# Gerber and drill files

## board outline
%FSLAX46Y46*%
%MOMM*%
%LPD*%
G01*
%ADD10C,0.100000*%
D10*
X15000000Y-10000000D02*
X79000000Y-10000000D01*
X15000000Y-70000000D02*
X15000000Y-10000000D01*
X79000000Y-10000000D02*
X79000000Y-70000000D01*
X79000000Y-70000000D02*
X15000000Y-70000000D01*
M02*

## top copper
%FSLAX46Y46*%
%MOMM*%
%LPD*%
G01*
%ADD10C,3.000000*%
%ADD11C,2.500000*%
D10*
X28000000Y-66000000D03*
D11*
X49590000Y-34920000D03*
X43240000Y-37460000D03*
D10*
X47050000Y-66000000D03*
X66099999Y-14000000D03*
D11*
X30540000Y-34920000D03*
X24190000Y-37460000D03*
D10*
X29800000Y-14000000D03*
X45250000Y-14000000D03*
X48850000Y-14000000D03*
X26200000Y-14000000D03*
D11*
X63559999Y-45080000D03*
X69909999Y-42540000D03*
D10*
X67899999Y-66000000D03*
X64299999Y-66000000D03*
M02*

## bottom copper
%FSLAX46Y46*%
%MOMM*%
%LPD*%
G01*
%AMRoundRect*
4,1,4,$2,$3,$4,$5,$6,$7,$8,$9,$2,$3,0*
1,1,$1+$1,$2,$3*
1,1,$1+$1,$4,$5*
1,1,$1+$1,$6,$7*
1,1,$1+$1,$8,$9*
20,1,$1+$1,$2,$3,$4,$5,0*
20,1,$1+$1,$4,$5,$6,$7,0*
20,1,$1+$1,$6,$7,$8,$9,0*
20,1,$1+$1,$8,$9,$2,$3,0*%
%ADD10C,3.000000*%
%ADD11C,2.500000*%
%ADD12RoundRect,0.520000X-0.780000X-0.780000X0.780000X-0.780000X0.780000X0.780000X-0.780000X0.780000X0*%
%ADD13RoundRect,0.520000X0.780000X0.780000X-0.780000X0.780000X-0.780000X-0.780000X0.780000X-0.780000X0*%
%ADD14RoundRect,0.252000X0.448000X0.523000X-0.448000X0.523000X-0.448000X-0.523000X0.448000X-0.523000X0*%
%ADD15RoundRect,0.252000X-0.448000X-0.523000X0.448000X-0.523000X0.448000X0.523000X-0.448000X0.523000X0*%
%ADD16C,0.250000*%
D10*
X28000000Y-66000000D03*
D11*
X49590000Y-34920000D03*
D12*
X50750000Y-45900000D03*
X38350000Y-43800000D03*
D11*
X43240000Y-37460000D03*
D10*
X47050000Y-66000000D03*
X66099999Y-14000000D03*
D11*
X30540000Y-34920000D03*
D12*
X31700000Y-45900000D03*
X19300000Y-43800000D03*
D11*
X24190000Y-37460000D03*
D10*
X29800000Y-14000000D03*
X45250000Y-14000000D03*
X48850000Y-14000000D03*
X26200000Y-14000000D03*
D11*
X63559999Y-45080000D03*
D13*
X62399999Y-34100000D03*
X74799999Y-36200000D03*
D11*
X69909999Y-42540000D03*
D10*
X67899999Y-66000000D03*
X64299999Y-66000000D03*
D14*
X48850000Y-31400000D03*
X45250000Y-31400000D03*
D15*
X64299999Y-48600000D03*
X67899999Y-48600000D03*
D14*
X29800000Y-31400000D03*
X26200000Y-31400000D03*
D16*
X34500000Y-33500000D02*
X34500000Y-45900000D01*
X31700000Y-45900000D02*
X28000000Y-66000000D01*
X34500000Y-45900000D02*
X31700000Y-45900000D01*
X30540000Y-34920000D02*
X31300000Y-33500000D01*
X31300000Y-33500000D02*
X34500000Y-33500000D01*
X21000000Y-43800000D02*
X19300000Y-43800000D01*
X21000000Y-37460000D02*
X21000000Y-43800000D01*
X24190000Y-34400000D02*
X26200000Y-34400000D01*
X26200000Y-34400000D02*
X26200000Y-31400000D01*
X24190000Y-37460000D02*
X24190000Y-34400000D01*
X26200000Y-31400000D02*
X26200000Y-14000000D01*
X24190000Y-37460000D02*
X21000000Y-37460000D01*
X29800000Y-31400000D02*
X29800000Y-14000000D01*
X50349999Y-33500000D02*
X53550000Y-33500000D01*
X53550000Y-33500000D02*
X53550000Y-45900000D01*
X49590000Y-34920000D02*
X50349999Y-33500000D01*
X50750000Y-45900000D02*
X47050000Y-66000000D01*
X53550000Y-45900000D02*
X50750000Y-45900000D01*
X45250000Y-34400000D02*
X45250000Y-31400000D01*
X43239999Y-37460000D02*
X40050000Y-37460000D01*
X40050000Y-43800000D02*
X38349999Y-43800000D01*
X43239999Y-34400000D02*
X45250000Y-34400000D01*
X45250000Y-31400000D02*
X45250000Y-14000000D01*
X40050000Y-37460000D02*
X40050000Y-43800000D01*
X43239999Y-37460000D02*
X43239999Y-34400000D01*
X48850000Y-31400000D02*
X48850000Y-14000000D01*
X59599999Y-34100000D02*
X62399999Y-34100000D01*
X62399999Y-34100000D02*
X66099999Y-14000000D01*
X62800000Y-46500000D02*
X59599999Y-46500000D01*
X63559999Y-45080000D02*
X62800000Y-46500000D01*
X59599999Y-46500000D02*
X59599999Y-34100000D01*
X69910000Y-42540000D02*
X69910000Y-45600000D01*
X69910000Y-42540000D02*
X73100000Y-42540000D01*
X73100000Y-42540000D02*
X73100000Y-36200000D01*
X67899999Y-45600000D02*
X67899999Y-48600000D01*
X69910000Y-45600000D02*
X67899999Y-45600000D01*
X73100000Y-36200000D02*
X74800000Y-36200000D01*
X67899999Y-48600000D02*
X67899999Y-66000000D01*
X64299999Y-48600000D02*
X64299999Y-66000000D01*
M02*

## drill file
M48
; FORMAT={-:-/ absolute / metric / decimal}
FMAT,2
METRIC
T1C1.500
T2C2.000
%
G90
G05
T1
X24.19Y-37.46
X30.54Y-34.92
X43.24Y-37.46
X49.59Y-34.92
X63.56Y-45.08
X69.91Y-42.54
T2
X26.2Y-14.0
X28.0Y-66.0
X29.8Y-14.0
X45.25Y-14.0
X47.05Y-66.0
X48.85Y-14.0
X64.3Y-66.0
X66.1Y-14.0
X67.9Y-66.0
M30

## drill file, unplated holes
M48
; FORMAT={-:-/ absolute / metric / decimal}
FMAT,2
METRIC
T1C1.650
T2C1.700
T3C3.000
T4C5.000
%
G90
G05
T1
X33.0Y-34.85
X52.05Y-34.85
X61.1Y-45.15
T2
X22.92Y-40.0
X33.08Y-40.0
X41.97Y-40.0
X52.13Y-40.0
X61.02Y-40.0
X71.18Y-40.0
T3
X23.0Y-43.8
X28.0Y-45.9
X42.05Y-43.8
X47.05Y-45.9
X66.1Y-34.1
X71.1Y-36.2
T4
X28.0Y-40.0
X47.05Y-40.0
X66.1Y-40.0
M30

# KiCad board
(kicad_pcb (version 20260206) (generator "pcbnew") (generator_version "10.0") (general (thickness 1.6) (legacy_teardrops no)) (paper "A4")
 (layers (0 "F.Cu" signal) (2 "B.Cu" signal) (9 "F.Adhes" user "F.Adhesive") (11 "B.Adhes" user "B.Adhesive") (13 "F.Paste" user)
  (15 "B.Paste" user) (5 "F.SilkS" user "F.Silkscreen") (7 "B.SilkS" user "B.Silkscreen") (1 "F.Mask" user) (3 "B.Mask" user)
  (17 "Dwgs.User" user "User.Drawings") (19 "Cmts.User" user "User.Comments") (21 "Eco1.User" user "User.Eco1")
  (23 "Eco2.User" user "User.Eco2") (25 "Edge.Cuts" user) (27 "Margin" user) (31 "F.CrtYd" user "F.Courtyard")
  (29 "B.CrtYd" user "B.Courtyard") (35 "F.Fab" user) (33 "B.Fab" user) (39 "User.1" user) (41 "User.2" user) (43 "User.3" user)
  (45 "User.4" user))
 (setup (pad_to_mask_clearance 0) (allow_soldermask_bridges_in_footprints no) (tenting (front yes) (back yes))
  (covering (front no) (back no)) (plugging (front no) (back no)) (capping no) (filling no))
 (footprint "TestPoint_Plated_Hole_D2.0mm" (layer "F.Cu") (at 28 66)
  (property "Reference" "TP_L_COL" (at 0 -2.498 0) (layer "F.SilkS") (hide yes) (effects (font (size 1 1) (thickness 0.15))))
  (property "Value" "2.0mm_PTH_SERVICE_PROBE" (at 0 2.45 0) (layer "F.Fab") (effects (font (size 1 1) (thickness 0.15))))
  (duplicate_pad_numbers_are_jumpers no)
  (pad "1" thru_hole circle (at 0 0) (size 3 3) (drill 2) (layers "*.Cu" "*.Mask") (remove_unused_layers no) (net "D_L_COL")))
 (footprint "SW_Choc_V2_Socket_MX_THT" (layer "F.Cu") (at 47.05 40)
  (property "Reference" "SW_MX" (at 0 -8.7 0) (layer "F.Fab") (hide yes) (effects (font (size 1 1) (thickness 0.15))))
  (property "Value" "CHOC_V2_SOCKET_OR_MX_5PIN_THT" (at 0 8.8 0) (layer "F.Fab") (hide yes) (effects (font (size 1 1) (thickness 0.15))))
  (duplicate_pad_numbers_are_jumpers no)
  (pad "" np_thru_hole circle (at -5.08 0) (size 1.7 1.7) (drill 1.7) (layers "*.Cu" "*.Mask"))
  (pad "" np_thru_hole circle (at -5 3.8) (size 3 3) (drill 3) (layers "*.Cu" "*.Mask"))
  (pad "" np_thru_hole circle (at 0 0) (size 5 5) (drill 5) (layers "*.Cu" "*.Mask"))
  (pad "" np_thru_hole circle (at 0 5.9) (size 3 3) (drill 3) (layers "*.Cu" "*.Mask"))
  (pad "" np_thru_hole circle (at 5 -5.15) (size 1.65 1.65) (drill 1.65) (layers "*.Cu" "*.Mask"))
  (pad "" np_thru_hole circle (at 5.08 0) (size 1.7 1.7) (drill 1.7) (layers "*.Cu" "*.Mask"))
  (pad "1" thru_hole circle (at 2.54 -5.08) (size 2.5 2.5) (drill 1.5) (layers "*.Cu" "*.Mask") (remove_unused_layers no) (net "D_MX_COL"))
  (pad "1" smd roundrect (at 3.7 5.9) (size 2.6 2.6) (layers "B.Cu" "B.Mask" "B.Paste") (roundrect_rratio 0.2) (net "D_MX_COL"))
  (pad "2" smd roundrect (at -8.7 3.8) (size 2.6 2.6) (layers "B.Cu" "B.Mask" "B.Paste") (roundrect_rratio 0.2) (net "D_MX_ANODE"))
  (pad "2" thru_hole circle (at -3.81 -2.54) (size 2.5 2.5) (drill 1.5) (layers "*.Cu" "*.Mask") (remove_unused_layers no)
   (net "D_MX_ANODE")))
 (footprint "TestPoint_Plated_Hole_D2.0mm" (layer "F.Cu") (at 47.05 66)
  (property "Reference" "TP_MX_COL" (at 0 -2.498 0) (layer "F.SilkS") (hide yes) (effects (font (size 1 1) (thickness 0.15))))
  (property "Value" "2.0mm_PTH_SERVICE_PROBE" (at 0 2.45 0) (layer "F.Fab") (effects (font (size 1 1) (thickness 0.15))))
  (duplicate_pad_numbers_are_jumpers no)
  (pad "1" thru_hole circle (at 0 0) (size 3 3) (drill 2) (layers "*.Cu" "*.Mask") (remove_unused_layers no) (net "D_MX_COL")))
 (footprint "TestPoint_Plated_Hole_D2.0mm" (layer "F.Cu") (at 66.099999 14)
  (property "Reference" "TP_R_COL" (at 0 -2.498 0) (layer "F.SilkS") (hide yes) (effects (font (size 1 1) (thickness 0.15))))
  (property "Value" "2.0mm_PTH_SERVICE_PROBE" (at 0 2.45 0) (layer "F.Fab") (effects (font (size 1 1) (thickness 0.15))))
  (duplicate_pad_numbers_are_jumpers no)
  (pad "1" thru_hole circle (at 0 0) (size 3 3) (drill 2) (layers "*.Cu" "*.Mask") (remove_unused_layers no) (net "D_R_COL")))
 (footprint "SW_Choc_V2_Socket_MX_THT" (layer "F.Cu") (at 28 40)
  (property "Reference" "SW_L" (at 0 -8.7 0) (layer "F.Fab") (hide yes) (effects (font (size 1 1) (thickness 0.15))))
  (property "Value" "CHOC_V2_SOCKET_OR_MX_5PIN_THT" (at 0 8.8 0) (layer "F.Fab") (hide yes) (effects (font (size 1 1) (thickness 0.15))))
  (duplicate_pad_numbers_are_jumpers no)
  (pad "" np_thru_hole circle (at -5.08 0) (size 1.7 1.7) (drill 1.7) (layers "*.Cu" "*.Mask"))
  (pad "" np_thru_hole circle (at -5 3.8) (size 3 3) (drill 3) (layers "*.Cu" "*.Mask"))
  (pad "" np_thru_hole circle (at 0 0) (size 5 5) (drill 5) (layers "*.Cu" "*.Mask"))
  (pad "" np_thru_hole circle (at 0 5.9) (size 3 3) (drill 3) (layers "*.Cu" "*.Mask"))
  (pad "" np_thru_hole circle (at 5 -5.15) (size 1.65 1.65) (drill 1.65) (layers "*.Cu" "*.Mask"))
  (pad "" np_thru_hole circle (at 5.08 0) (size 1.7 1.7) (drill 1.7) (layers "*.Cu" "*.Mask"))
  (pad "1" thru_hole circle (at 2.54 -5.08) (size 2.5 2.5) (drill 1.5) (layers "*.Cu" "*.Mask") (remove_unused_layers no) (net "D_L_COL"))
  (pad "1" smd roundrect (at 3.7 5.9) (size 2.6 2.6) (layers "B.Cu" "B.Mask" "B.Paste") (roundrect_rratio 0.2) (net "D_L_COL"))
  (pad "2" smd roundrect (at -8.7 3.8) (size 2.6 2.6) (layers "B.Cu" "B.Mask" "B.Paste") (roundrect_rratio 0.2) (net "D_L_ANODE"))
  (pad "2" thru_hole circle (at -3.81 -2.54) (size 2.5 2.5) (drill 1.5) (layers "*.Cu" "*.Mask") (remove_unused_layers no) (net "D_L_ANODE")))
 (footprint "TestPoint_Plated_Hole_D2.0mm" (layer "F.Cu") (at 29.8 14)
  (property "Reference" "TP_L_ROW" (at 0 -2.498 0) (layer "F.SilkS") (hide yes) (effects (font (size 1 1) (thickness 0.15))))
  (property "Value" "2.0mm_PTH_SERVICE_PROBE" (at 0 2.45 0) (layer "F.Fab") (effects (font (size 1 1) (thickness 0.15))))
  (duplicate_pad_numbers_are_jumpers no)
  (pad "1" thru_hole circle (at 0 0) (size 3 3) (drill 2) (layers "*.Cu" "*.Mask") (remove_unused_layers no) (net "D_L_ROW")))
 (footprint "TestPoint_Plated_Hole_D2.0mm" (layer "F.Cu") (at 45.25 14)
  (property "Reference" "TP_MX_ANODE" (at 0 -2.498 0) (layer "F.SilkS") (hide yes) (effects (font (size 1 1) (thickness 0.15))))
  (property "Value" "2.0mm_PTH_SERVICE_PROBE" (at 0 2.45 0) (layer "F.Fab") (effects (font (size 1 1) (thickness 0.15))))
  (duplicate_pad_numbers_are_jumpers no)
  (pad "1" thru_hole circle (at 0 0) (size 3 3) (drill 2) (layers "*.Cu" "*.Mask") (remove_unused_layers no) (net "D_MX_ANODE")))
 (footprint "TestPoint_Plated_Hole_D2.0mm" (layer "F.Cu") (at 48.85 14)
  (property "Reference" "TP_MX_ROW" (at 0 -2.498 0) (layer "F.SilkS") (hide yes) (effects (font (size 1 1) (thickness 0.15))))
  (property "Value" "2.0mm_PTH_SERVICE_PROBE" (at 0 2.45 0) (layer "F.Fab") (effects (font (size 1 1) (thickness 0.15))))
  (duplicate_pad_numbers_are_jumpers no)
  (pad "1" thru_hole circle (at 0 0) (size 3 3) (drill 2) (layers "*.Cu" "*.Mask") (remove_unused_layers no) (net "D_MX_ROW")))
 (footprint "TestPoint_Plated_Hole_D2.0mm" (layer "F.Cu") (at 26.2 14)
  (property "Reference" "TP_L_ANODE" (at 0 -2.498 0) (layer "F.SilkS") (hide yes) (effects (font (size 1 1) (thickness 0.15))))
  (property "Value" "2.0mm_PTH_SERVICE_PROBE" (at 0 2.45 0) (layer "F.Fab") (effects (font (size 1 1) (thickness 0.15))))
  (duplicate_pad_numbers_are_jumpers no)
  (pad "1" thru_hole circle (at 0 0) (size 3 3) (drill 2) (layers "*.Cu" "*.Mask") (remove_unused_layers no) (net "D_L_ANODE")))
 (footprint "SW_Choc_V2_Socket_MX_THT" (layer "F.Cu") (at 66.099999 40 180)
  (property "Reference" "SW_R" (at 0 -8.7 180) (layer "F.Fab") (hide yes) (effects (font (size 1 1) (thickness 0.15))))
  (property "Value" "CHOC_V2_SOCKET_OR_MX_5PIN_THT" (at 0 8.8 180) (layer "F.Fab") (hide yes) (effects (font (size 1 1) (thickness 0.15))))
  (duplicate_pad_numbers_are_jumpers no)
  (pad "" np_thru_hole circle (at -5.08 0 180) (size 1.7 1.7) (drill 1.7) (layers "*.Cu" "*.Mask"))
  (pad "" np_thru_hole circle (at -5 3.8 180) (size 3 3) (drill 3) (layers "*.Cu" "*.Mask"))
  (pad "" np_thru_hole circle (at 0 0 180) (size 5 5) (drill 5) (layers "*.Cu" "*.Mask"))
  (pad "" np_thru_hole circle (at 0 5.9 180) (size 3 3) (drill 3) (layers "*.Cu" "*.Mask"))
  (pad "" np_thru_hole circle (at 5 -5.15 180) (size 1.65 1.65) (drill 1.65) (layers "*.Cu" "*.Mask"))
  (pad "" np_thru_hole circle (at 5.08 0 180) (size 1.7 1.7) (drill 1.7) (layers "*.Cu" "*.Mask"))
  (pad "1" thru_hole circle (at 2.54 -5.08 180) (size 2.5 2.5) (drill 1.5) (layers "*.Cu" "*.Mask") (remove_unused_layers no)
   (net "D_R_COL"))
  (pad "1" smd roundrect (at 3.7 5.9 180) (size 2.6 2.6) (layers "B.Cu" "B.Mask" "B.Paste") (roundrect_rratio 0.2) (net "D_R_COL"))
  (pad "2" smd roundrect (at -8.7 3.8 180) (size 2.6 2.6) (layers "B.Cu" "B.Mask" "B.Paste") (roundrect_rratio 0.2) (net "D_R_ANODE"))
  (pad "2" thru_hole circle (at -3.81 -2.54 180) (size 2.5 2.5) (drill 1.5) (layers "*.Cu" "*.Mask") (remove_unused_layers no)
   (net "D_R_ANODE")))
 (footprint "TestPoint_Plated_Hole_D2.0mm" (layer "F.Cu") (at 67.899999 66)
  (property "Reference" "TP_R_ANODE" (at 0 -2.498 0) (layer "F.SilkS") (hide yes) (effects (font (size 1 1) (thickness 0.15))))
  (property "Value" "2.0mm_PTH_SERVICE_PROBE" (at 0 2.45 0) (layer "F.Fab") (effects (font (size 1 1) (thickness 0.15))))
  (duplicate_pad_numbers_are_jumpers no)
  (pad "1" thru_hole circle (at 0 0) (size 3 3) (drill 2) (layers "*.Cu" "*.Mask") (remove_unused_layers no) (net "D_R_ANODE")))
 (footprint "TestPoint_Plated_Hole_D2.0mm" (layer "F.Cu") (at 64.299999 66)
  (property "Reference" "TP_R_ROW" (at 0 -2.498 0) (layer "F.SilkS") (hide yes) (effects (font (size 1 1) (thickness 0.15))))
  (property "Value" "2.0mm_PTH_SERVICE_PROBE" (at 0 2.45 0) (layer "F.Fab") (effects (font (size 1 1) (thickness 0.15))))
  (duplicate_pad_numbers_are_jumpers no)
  (pad "1" thru_hole circle (at 0 0) (size 3 3) (drill 2) (layers "*.Cu" "*.Mask") (remove_unused_layers no) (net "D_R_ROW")))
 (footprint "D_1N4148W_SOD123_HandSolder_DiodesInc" (layer "B.Cu") (at 47.05 31.4 180)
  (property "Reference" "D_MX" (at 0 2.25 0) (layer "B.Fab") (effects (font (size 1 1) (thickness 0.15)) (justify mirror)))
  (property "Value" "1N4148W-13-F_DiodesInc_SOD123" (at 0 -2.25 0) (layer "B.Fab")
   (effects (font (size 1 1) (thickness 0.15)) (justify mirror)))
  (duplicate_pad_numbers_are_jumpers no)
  (pad "1" smd roundrect (at -1.8 0 180) (size 1.4 1.55) (layers "B.Cu" "B.Mask" "B.Paste") (roundrect_rratio 0.18) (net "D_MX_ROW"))
  (pad "2" smd roundrect (at 1.8 0 180) (size 1.4 1.55) (layers "B.Cu" "B.Mask" "B.Paste") (roundrect_rratio 0.18) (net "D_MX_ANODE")))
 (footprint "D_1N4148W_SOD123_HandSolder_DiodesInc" (layer "B.Cu") (at 66.099999 48.6)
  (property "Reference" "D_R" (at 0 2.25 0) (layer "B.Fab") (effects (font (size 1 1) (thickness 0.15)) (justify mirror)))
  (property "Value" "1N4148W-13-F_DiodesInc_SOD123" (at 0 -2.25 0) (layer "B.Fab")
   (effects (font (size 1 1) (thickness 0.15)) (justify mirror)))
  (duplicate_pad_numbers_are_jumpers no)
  (pad "1" smd roundrect (at -1.8 0) (size 1.4 1.55) (layers "B.Cu" "B.Mask" "B.Paste") (roundrect_rratio 0.18) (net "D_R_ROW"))
  (pad "2" smd roundrect (at 1.8 0) (size 1.4 1.55) (layers "B.Cu" "B.Mask" "B.Paste") (roundrect_rratio 0.18) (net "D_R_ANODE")))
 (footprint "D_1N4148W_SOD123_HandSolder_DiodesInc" (layer "B.Cu") (at 28 31.4 180)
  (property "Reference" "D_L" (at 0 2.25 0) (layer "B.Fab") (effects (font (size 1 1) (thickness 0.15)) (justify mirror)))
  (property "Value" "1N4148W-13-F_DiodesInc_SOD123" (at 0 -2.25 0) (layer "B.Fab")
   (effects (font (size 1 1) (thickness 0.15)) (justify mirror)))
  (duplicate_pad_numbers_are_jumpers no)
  (pad "1" smd roundrect (at -1.8 0 180) (size 1.4 1.55) (layers "B.Cu" "B.Mask" "B.Paste") (roundrect_rratio 0.18) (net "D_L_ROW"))
  (pad "2" smd roundrect (at 1.8 0 180) (size 1.4 1.55) (layers "B.Cu" "B.Mask" "B.Paste") (roundrect_rratio 0.18) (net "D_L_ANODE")))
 (gr_line (start 15 10) (end 79 10) (stroke (width 0.1) (type default)) (layer "Edge.Cuts"))
 (gr_line (start 15 70) (end 15 10) (stroke (width 0.1) (type default)) (layer "Edge.Cuts"))
 (gr_line (start 79 10) (end 79 70) (stroke (width 0.1) (type default)) (layer "Edge.Cuts"))
 (gr_line (start 79 70) (end 15 70) (stroke (width 0.1) (type default)) (layer "Edge.Cuts"))
 (segment (start 34.5 33.5) (end 34.5 45.9) (width 0.25) (layer "B.Cu") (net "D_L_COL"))
 (segment (start 31.7 45.9) (end 28 66) (width 0.25) (layer "B.Cu") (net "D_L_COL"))
 (segment (start 34.5 45.9) (end 31.7 45.9) (width 0.25) (layer "B.Cu") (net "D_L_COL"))
 (segment (start 30.54 34.92) (end 31.3 33.5) (width 0.25) (layer "B.Cu") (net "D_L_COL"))
 (segment (start 31.3 33.5) (end 34.5 33.5) (width 0.25) (layer "B.Cu") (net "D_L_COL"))
 (segment (start 21 43.8) (end 19.3 43.8) (width 0.25) (layer "B.Cu") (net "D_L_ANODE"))
 (segment (start 21 37.46) (end 21 43.8) (width 0.25) (layer "B.Cu") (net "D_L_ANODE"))
 (segment (start 24.19 34.4) (end 26.2 34.4) (width 0.25) (layer "B.Cu") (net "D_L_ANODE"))
 (segment (start 26.2 34.4) (end 26.2 31.4) (width 0.25) (layer "B.Cu") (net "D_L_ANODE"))
 (segment (start 24.19 37.46) (end 24.19 34.4) (width 0.25) (layer "B.Cu") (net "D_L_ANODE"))
 (segment (start 26.2 31.4) (end 26.2 14) (width 0.25) (layer "B.Cu") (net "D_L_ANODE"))
 (segment (start 24.19 37.46) (end 21 37.46) (width 0.25) (layer "B.Cu") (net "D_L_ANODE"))
 (segment (start 29.8 31.4) (end 29.8 14) (width 0.25) (layer "B.Cu") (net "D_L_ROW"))
 (segment (start 50.349999 33.5) (end 53.55 33.5) (width 0.25) (layer "B.Cu") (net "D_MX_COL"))
 (segment (start 53.55 33.5) (end 53.55 45.9) (width 0.25) (layer "B.Cu") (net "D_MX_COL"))
 (segment (start 49.59 34.92) (end 50.349999 33.5) (width 0.25) (layer "B.Cu") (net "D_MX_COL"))
 (segment (start 50.75 45.9) (end 47.05 66) (width 0.25) (layer "B.Cu") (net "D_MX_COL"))
 (segment (start 53.55 45.9) (end 50.75 45.9) (width 0.25) (layer "B.Cu") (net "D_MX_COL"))
 (segment (start 45.25 34.4) (end 45.25 31.4) (width 0.25) (layer "B.Cu") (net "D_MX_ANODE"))
 (segment (start 43.239999 37.46) (end 40.05 37.46) (width 0.25) (layer "B.Cu") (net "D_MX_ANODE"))
 (segment (start 40.05 43.8) (end 38.349999 43.8) (width 0.25) (layer "B.Cu") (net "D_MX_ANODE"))
 (segment (start 43.239999 34.4) (end 45.25 34.4) (width 0.25) (layer "B.Cu") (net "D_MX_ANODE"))
 (segment (start 45.25 31.4) (end 45.25 14) (width 0.25) (layer "B.Cu") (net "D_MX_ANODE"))
 (segment (start 40.05 37.46) (end 40.05 43.8) (width 0.25) (layer "B.Cu") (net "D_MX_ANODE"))
 (segment (start 43.239999 37.46) (end 43.239999 34.4) (width 0.25) (layer "B.Cu") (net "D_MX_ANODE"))
 (segment (start 48.85 31.4) (end 48.85 14) (width 0.25) (layer "B.Cu") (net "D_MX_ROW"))
 (segment (start 59.599999 34.1) (end 62.399999 34.1) (width 0.25) (layer "B.Cu") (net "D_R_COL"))
 (segment (start 62.399999 34.1) (end 66.099999 14) (width 0.25) (layer "B.Cu") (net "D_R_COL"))
 (segment (start 62.8 46.5) (end 59.599999 46.5) (width 0.25) (layer "B.Cu") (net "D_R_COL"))
 (segment (start 63.559999 45.08) (end 62.8 46.5) (width 0.25) (layer "B.Cu") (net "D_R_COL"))
 (segment (start 59.599999 46.5) (end 59.599999 34.1) (width 0.25) (layer "B.Cu") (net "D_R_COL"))
 (segment (start 69.91 42.54) (end 69.91 45.6) (width 0.25) (layer "B.Cu") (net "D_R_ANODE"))
 (segment (start 69.91 42.54) (end 73.1 42.54) (width 0.25) (layer "B.Cu") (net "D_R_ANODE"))
 (segment (start 73.1 42.54) (end 73.1 36.2) (width 0.25) (layer "B.Cu") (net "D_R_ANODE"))
 (segment (start 67.899999 45.6) (end 67.899999 48.6) (width 0.25) (layer "B.Cu") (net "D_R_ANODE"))
 (segment (start 69.91 45.6) (end 67.899999 45.6) (width 0.25) (layer "B.Cu") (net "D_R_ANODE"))
 (segment (start 73.1 36.2) (end 74.8 36.2) (width 0.25) (layer "B.Cu") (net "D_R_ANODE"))
 (segment (start 67.899999 48.6) (end 67.899999 66) (width 0.25) (layer "B.Cu") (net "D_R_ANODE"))
 (segment (start 64.299999 48.6) (end 64.299999 66) (width 0.25) (layer "B.Cu") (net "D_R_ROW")))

